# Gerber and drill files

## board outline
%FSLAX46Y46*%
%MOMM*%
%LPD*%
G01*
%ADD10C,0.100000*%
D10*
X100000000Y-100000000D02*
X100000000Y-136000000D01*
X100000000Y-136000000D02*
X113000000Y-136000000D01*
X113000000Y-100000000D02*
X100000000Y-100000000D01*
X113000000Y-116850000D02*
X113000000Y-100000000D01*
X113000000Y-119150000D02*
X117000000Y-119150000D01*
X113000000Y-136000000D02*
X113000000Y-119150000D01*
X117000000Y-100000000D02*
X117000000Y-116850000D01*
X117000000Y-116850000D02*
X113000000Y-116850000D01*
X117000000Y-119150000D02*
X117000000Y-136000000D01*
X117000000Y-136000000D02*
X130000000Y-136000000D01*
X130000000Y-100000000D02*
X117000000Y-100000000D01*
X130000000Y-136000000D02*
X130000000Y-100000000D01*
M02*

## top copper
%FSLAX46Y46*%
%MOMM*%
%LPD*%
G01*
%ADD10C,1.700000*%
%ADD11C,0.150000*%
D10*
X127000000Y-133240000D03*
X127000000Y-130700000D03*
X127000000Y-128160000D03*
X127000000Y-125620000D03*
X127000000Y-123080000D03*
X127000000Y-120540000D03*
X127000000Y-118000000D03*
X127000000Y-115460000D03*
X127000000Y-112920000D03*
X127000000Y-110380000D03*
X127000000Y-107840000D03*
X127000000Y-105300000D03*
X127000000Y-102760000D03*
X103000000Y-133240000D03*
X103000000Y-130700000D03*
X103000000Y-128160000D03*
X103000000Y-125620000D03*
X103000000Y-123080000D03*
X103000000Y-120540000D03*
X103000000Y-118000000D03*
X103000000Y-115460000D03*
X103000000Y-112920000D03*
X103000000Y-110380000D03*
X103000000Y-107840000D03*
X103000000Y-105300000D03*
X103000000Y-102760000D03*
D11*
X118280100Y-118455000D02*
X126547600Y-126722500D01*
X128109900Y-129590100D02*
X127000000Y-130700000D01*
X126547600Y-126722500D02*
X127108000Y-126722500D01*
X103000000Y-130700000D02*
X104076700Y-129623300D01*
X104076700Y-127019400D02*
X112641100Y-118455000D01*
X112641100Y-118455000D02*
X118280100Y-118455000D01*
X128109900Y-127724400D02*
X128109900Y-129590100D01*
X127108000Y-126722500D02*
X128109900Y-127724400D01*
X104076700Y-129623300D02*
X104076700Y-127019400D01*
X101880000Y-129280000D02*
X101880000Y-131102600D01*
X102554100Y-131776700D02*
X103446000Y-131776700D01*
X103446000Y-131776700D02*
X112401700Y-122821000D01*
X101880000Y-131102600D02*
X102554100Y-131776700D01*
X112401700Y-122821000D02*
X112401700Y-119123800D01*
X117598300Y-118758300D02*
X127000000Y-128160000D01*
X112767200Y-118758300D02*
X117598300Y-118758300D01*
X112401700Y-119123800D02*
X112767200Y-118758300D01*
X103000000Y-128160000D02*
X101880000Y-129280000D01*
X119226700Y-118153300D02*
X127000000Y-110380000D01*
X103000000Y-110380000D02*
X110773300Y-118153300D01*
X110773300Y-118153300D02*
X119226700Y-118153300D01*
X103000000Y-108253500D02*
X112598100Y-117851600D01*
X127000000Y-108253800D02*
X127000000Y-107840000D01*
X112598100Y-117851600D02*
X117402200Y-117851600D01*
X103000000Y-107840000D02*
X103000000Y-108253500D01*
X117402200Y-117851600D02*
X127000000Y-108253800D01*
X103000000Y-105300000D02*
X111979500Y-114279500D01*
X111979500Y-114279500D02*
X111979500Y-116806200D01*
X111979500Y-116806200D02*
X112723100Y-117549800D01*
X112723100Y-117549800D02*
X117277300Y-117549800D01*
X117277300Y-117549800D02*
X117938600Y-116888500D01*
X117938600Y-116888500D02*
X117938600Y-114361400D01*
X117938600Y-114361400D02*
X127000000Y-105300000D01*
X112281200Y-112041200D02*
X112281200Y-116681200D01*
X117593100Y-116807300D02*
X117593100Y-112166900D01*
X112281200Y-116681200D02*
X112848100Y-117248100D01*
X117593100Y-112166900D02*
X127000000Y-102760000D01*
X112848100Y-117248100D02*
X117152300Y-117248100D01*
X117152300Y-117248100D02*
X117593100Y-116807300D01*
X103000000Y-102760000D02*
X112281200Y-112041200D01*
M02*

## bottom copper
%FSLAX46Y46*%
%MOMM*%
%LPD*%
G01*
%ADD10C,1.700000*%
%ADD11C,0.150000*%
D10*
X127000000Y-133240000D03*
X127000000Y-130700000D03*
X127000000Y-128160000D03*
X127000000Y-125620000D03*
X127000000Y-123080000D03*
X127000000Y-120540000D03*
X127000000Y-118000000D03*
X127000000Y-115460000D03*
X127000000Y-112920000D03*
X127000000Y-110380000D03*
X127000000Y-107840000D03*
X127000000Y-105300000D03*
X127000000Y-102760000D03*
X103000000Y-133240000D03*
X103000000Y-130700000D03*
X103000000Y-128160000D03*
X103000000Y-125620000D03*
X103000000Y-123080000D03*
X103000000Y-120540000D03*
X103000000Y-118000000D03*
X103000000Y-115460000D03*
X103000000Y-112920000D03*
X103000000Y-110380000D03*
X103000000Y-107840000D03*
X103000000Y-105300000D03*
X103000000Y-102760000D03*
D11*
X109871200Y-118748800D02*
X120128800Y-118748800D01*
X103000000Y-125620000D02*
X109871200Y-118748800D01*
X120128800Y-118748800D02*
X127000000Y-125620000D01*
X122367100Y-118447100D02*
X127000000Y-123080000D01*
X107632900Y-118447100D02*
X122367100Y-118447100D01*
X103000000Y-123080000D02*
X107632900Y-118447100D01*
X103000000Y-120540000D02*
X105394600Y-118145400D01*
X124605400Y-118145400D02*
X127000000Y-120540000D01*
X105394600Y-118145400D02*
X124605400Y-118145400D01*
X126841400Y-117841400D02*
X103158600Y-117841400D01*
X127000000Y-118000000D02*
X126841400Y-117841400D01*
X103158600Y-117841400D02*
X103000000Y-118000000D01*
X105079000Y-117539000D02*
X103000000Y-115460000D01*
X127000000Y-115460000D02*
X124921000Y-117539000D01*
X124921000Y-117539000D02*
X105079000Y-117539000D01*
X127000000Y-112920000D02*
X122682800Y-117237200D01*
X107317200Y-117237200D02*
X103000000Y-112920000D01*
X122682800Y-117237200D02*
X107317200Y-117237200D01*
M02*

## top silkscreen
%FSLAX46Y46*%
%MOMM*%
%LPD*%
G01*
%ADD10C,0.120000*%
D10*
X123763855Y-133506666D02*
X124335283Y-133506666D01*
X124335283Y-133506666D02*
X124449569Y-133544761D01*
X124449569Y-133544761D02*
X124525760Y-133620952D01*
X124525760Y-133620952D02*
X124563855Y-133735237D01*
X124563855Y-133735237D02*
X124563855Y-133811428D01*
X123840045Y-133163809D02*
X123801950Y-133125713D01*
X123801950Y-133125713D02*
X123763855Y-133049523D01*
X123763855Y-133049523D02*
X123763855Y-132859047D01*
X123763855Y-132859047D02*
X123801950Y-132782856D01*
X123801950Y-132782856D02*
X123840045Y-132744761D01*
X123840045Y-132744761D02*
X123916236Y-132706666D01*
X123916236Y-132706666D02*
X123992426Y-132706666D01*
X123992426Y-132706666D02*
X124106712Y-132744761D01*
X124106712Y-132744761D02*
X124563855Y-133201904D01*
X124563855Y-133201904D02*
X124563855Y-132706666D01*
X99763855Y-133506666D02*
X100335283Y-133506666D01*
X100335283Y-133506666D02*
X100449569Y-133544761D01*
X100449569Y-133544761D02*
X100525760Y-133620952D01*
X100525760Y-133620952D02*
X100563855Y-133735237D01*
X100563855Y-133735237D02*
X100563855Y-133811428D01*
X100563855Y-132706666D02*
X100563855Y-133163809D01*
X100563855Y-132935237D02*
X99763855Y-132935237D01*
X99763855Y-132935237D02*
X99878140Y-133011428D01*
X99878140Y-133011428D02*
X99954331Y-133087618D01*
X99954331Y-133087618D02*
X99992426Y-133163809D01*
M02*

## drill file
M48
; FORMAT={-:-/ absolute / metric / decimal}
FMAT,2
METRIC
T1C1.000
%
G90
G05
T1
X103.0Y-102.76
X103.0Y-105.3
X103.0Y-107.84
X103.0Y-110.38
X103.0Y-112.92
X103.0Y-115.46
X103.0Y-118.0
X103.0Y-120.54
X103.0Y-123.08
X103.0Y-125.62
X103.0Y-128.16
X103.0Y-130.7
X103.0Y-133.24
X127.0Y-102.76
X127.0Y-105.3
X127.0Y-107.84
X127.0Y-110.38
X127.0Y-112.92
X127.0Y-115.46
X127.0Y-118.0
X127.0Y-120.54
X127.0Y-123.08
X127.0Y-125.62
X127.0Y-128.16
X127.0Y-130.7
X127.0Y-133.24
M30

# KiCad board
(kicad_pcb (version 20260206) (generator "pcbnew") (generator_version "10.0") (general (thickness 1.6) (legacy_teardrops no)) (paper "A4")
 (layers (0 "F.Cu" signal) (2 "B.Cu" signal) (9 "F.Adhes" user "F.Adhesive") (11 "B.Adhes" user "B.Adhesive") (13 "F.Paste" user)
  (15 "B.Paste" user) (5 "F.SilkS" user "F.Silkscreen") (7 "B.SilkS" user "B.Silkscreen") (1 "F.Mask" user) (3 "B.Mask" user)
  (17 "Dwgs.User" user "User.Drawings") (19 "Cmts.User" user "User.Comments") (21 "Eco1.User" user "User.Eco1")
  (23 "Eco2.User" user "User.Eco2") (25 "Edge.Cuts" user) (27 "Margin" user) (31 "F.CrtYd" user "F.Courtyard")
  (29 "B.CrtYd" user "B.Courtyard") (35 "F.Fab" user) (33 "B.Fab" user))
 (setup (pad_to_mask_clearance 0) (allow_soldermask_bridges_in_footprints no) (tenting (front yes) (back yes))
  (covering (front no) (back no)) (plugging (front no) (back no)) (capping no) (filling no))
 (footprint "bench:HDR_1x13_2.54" (layer "F.Cu") (at 127 133.24 90)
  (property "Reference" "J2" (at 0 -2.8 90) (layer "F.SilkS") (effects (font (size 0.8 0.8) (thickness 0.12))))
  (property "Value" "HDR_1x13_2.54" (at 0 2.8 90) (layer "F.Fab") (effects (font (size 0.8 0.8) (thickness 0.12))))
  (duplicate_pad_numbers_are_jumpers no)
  (pad "1" thru_hole circle (at 0 0 90) (size 1.7 1.7) (drill 1) (layers "*.Cu" "*.Mask") (remove_unused_layers no) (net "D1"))
  (pad "2" thru_hole circle (at 2.54 0 90) (size 1.7 1.7) (drill 1) (layers "*.Cu" "*.Mask") (remove_unused_layers no) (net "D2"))
  (pad "3" thru_hole circle (at 5.08 0 90) (size 1.7 1.7) (drill 1) (layers "*.Cu" "*.Mask") (remove_unused_layers no) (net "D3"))
  (pad "4" thru_hole circle (at 7.62 0 90) (size 1.7 1.7) (drill 1) (layers "*.Cu" "*.Mask") (remove_unused_layers no) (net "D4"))
  (pad "5" thru_hole circle (at 10.16 0 90) (size 1.7 1.7) (drill 1) (layers "*.Cu" "*.Mask") (remove_unused_layers no) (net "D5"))
  (pad "6" thru_hole circle (at 12.7 0 90) (size 1.7 1.7) (drill 1) (layers "*.Cu" "*.Mask") (remove_unused_layers no) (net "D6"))
  (pad "7" thru_hole circle (at 15.24 0 90) (size 1.7 1.7) (drill 1) (layers "*.Cu" "*.Mask") (remove_unused_layers no) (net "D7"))
  (pad "8" thru_hole circle (at 17.78 0 90) (size 1.7 1.7) (drill 1) (layers "*.Cu" "*.Mask") (remove_unused_layers no) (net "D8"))
  (pad "9" thru_hole circle (at 20.32 0 90) (size 1.7 1.7) (drill 1) (layers "*.Cu" "*.Mask") (remove_unused_layers no) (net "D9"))
  (pad "10" thru_hole circle (at 22.86 0 90) (size 1.7 1.7) (drill 1) (layers "*.Cu" "*.Mask") (remove_unused_layers no) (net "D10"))
  (pad "11" thru_hole circle (at 25.4 0 90) (size 1.7 1.7) (drill 1) (layers "*.Cu" "*.Mask") (remove_unused_layers no) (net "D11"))
  (pad "12" thru_hole circle (at 27.94 0 90) (size 1.7 1.7) (drill 1) (layers "*.Cu" "*.Mask") (remove_unused_layers no) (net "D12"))
  (pad "13" thru_hole circle (at 30.48 0 90) (size 1.7 1.7) (drill 1) (layers "*.Cu" "*.Mask") (remove_unused_layers no) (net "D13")))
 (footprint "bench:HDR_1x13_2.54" (layer "F.Cu") (at 103 133.24 90)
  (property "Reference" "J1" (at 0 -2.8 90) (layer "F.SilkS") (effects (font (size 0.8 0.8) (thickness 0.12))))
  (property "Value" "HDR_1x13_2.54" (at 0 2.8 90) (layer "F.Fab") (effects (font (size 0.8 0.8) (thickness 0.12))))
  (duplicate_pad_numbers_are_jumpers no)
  (pad "1" thru_hole circle (at 0 0 90) (size 1.7 1.7) (drill 1) (layers "*.Cu" "*.Mask") (remove_unused_layers no) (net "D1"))
  (pad "2" thru_hole circle (at 2.54 0 90) (size 1.7 1.7) (drill 1) (layers "*.Cu" "*.Mask") (remove_unused_layers no) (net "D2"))
  (pad "3" thru_hole circle (at 5.08 0 90) (size 1.7 1.7) (drill 1) (layers "*.Cu" "*.Mask") (remove_unused_layers no) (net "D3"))
  (pad "4" thru_hole circle (at 7.62 0 90) (size 1.7 1.7) (drill 1) (layers "*.Cu" "*.Mask") (remove_unused_layers no) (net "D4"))
  (pad "5" thru_hole circle (at 10.16 0 90) (size 1.7 1.7) (drill 1) (layers "*.Cu" "*.Mask") (remove_unused_layers no) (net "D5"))
  (pad "6" thru_hole circle (at 12.7 0 90) (size 1.7 1.7) (drill 1) (layers "*.Cu" "*.Mask") (remove_unused_layers no) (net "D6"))
  (pad "7" thru_hole circle (at 15.24 0 90) (size 1.7 1.7) (drill 1) (layers "*.Cu" "*.Mask") (remove_unused_layers no) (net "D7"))
  (pad "8" thru_hole circle (at 17.78 0 90) (size 1.7 1.7) (drill 1) (layers "*.Cu" "*.Mask") (remove_unused_layers no) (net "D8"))
  (pad "9" thru_hole circle (at 20.32 0 90) (size 1.7 1.7) (drill 1) (layers "*.Cu" "*.Mask") (remove_unused_layers no) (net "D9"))
  (pad "10" thru_hole circle (at 22.86 0 90) (size 1.7 1.7) (drill 1) (layers "*.Cu" "*.Mask") (remove_unused_layers no) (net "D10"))
  (pad "11" thru_hole circle (at 25.4 0 90) (size 1.7 1.7) (drill 1) (layers "*.Cu" "*.Mask") (remove_unused_layers no) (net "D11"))
  (pad "12" thru_hole circle (at 27.94 0 90) (size 1.7 1.7) (drill 1) (layers "*.Cu" "*.Mask") (remove_unused_layers no) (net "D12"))
  (pad "13" thru_hole circle (at 30.48 0 90) (size 1.7 1.7) (drill 1) (layers "*.Cu" "*.Mask") (remove_unused_layers no) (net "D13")))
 (gr_line (start 100 100) (end 100 136) (stroke (width 0.1) (type solid)) (layer "Edge.Cuts"))
 (gr_line (start 100 136) (end 113 136) (stroke (width 0.1) (type solid)) (layer "Edge.Cuts"))
 (gr_line (start 113 100) (end 100 100) (stroke (width 0.1) (type solid)) (layer "Edge.Cuts"))
 (gr_line (start 113 116.85) (end 113 100) (stroke (width 0.1) (type solid)) (layer "Edge.Cuts"))
 (gr_line (start 113 119.15) (end 117 119.15) (stroke (width 0.1) (type solid)) (layer "Edge.Cuts"))
 (gr_line (start 113 136) (end 113 119.15) (stroke (width 0.1) (type solid)) (layer "Edge.Cuts"))
 (gr_line (start 117 100) (end 117 116.85) (stroke (width 0.1) (type solid)) (layer "Edge.Cuts"))
 (gr_line (start 117 116.85) (end 113 116.85) (stroke (width 0.1) (type solid)) (layer "Edge.Cuts"))
 (gr_line (start 117 119.15) (end 117 136) (stroke (width 0.1) (type solid)) (layer "Edge.Cuts"))
 (gr_line (start 117 136) (end 130 136) (stroke (width 0.1) (type solid)) (layer "Edge.Cuts"))
 (gr_line (start 130 100) (end 117 100) (stroke (width 0.1) (type solid)) (layer "Edge.Cuts"))
 (gr_line (start 130 136) (end 130 100) (stroke (width 0.1) (type solid)) (layer "Edge.Cuts"))
 (segment (start 118.2801 118.455) (end 126.5476 126.7225) (width 0.15) (layer "F.Cu") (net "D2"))
 (segment (start 128.1099 129.5901) (end 127 130.7) (width 0.15) (layer "F.Cu") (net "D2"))
 (segment (start 126.5476 126.7225) (end 127.108 126.7225) (width 0.15) (layer "F.Cu") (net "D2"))
 (segment (start 103 130.7) (end 104.0767 129.6233) (width 0.15) (layer "F.Cu") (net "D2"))
 (segment (start 104.0767 127.0194) (end 112.6411 118.455) (width 0.15) (layer "F.Cu") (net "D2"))
 (segment (start 112.6411 118.455) (end 118.2801 118.455) (width 0.15) (layer "F.Cu") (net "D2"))
 (segment (start 128.1099 127.7244) (end 128.1099 129.5901) (width 0.15) (layer "F.Cu") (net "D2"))
 (segment (start 127.108 126.7225) (end 128.1099 127.7244) (width 0.15) (layer "F.Cu") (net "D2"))
 (segment (start 104.0767 129.6233) (end 104.0767 127.0194) (width 0.15) (layer "F.Cu") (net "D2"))
 (segment (start 101.88 129.28) (end 101.88 131.1026) (width 0.15) (layer "F.Cu") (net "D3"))
 (segment (start 102.5541 131.7767) (end 103.446 131.7767) (width 0.15) (layer "F.Cu") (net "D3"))
 (segment (start 103.446 131.7767) (end 112.4017 122.821) (width 0.15) (layer "F.Cu") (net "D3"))
 (segment (start 101.88 131.1026) (end 102.5541 131.7767) (width 0.15) (layer "F.Cu") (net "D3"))
 (segment (start 112.4017 122.821) (end 112.4017 119.1238) (width 0.15) (layer "F.Cu") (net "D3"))
 (segment (start 117.5983 118.7583) (end 127 128.16) (width 0.15) (layer "F.Cu") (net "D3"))
 (segment (start 112.7672 118.7583) (end 117.5983 118.7583) (width 0.15) (layer "F.Cu") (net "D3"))
 (segment (start 112.4017 119.1238) (end 112.7672 118.7583) (width 0.15) (layer "F.Cu") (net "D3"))
 (segment (start 103 128.16) (end 101.88 129.28) (width 0.15) (layer "F.Cu") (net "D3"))
 (segment (start 109.8712 118.7488) (end 120.1288 118.7488) (width 0.15) (layer "B.Cu") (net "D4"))
 (segment (start 103 125.62) (end 109.8712 118.7488) (width 0.15) (layer "B.Cu") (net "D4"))
 (segment (start 120.1288 118.7488) (end 127 125.62) (width 0.15) (layer "B.Cu") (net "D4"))
 (segment (start 122.3671 118.4471) (end 127 123.08) (width 0.15) (layer "B.Cu") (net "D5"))
 (segment (start 107.6329 118.4471) (end 122.3671 118.4471) (width 0.15) (layer "B.Cu") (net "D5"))
 (segment (start 103 123.08) (end 107.6329 118.4471) (width 0.15) (layer "B.Cu") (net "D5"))
 (segment (start 103 120.54) (end 105.3946 118.1454) (width 0.15) (layer "B.Cu") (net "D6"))
 (segment (start 124.6054 118.1454) (end 127 120.54) (width 0.15) (layer "B.Cu") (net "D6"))
 (segment (start 105.3946 118.1454) (end 124.6054 118.1454) (width 0.15) (layer "B.Cu") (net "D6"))
 (segment (start 126.8414 117.8414) (end 103.1586 117.8414) (width 0.15) (layer "B.Cu") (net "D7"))
 (segment (start 127 118) (end 126.8414 117.8414) (width 0.15) (layer "B.Cu") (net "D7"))
 (segment (start 103.1586 117.8414) (end 103 118) (width 0.15) (layer "B.Cu") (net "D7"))
 (segment (start 105.079 117.539) (end 103 115.46) (width 0.15) (layer "B.Cu") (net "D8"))
 (segment (start 127 115.46) (end 124.921 117.539) (width 0.15) (layer "B.Cu") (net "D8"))
 (segment (start 124.921 117.539) (end 105.079 117.539) (width 0.15) (layer "B.Cu") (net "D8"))
 (segment (start 127 112.92) (end 122.6828 117.2372) (width 0.15) (layer "B.Cu") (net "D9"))
 (segment (start 107.3172 117.2372) (end 103 112.92) (width 0.15) (layer "B.Cu") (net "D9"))
 (segment (start 122.6828 117.2372) (end 107.3172 117.2372) (width 0.15) (layer "B.Cu") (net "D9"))
 (segment (start 119.2267 118.1533) (end 127 110.38) (width 0.15) (layer "F.Cu") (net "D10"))
 (segment (start 103 110.38) (end 110.7733 118.1533) (width 0.15) (layer "F.Cu") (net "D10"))
 (segment (start 110.7733 118.1533) (end 119.2267 118.1533) (width 0.15) (layer "F.Cu") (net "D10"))
 (segment (start 103 108.2535) (end 112.5981 117.8516) (width 0.15) (layer "F.Cu") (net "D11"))
 (segment (start 127 108.2538) (end 127 107.84) (width 0.15) (layer "F.Cu") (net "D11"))
 (segment (start 112.5981 117.8516) (end 117.4022 117.8516) (width 0.15) (layer "F.Cu") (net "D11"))
 (segment (start 103 107.84) (end 103 108.2535) (width 0.15) (layer "F.Cu") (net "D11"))
 (segment (start 117.4022 117.8516) (end 127 108.2538) (width 0.15) (layer "F.Cu") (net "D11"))
 (segment (start 103 105.3) (end 111.9795 114.2795) (width 0.15) (layer "F.Cu") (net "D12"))
 (segment (start 111.9795 114.2795) (end 111.9795 116.8062) (width 0.15) (layer "F.Cu") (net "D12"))
 (segment (start 111.9795 116.8062) (end 112.7231 117.5498) (width 0.15) (layer "F.Cu") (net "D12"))
 (segment (start 112.7231 117.5498) (end 117.2773 117.5498) (width 0.15) (layer "F.Cu") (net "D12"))
 (segment (start 117.2773 117.5498) (end 117.9386 116.8885) (width 0.15) (layer "F.Cu") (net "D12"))
 (segment (start 117.9386 116.8885) (end 117.9386 114.3614) (width 0.15) (layer "F.Cu") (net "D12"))
 (segment (start 117.9386 114.3614) (end 127 105.3) (width 0.15) (layer "F.Cu") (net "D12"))
 (segment (start 112.2812 112.0412) (end 112.2812 116.6812) (width 0.15) (layer "F.Cu") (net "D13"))
 (segment (start 117.5931 116.8073) (end 117.5931 112.1669) (width 0.15) (layer "F.Cu") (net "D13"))
 (segment (start 112.2812 116.6812) (end 112.8481 117.2481) (width 0.15) (layer "F.Cu") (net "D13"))
 (segment (start 117.5931 112.1669) (end 127 102.76) (width 0.15) (layer "F.Cu") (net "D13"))
 (segment (start 112.8481 117.2481) (end 117.1523 117.2481) (width 0.15) (layer "F.Cu") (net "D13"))
 (segment (start 117.1523 117.2481) (end 117.5931 116.8073) (width 0.15) (layer "F.Cu") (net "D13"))
 (segment (start 103 102.76) (end 112.2812 112.0412) (width 0.15) (layer "F.Cu") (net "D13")))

